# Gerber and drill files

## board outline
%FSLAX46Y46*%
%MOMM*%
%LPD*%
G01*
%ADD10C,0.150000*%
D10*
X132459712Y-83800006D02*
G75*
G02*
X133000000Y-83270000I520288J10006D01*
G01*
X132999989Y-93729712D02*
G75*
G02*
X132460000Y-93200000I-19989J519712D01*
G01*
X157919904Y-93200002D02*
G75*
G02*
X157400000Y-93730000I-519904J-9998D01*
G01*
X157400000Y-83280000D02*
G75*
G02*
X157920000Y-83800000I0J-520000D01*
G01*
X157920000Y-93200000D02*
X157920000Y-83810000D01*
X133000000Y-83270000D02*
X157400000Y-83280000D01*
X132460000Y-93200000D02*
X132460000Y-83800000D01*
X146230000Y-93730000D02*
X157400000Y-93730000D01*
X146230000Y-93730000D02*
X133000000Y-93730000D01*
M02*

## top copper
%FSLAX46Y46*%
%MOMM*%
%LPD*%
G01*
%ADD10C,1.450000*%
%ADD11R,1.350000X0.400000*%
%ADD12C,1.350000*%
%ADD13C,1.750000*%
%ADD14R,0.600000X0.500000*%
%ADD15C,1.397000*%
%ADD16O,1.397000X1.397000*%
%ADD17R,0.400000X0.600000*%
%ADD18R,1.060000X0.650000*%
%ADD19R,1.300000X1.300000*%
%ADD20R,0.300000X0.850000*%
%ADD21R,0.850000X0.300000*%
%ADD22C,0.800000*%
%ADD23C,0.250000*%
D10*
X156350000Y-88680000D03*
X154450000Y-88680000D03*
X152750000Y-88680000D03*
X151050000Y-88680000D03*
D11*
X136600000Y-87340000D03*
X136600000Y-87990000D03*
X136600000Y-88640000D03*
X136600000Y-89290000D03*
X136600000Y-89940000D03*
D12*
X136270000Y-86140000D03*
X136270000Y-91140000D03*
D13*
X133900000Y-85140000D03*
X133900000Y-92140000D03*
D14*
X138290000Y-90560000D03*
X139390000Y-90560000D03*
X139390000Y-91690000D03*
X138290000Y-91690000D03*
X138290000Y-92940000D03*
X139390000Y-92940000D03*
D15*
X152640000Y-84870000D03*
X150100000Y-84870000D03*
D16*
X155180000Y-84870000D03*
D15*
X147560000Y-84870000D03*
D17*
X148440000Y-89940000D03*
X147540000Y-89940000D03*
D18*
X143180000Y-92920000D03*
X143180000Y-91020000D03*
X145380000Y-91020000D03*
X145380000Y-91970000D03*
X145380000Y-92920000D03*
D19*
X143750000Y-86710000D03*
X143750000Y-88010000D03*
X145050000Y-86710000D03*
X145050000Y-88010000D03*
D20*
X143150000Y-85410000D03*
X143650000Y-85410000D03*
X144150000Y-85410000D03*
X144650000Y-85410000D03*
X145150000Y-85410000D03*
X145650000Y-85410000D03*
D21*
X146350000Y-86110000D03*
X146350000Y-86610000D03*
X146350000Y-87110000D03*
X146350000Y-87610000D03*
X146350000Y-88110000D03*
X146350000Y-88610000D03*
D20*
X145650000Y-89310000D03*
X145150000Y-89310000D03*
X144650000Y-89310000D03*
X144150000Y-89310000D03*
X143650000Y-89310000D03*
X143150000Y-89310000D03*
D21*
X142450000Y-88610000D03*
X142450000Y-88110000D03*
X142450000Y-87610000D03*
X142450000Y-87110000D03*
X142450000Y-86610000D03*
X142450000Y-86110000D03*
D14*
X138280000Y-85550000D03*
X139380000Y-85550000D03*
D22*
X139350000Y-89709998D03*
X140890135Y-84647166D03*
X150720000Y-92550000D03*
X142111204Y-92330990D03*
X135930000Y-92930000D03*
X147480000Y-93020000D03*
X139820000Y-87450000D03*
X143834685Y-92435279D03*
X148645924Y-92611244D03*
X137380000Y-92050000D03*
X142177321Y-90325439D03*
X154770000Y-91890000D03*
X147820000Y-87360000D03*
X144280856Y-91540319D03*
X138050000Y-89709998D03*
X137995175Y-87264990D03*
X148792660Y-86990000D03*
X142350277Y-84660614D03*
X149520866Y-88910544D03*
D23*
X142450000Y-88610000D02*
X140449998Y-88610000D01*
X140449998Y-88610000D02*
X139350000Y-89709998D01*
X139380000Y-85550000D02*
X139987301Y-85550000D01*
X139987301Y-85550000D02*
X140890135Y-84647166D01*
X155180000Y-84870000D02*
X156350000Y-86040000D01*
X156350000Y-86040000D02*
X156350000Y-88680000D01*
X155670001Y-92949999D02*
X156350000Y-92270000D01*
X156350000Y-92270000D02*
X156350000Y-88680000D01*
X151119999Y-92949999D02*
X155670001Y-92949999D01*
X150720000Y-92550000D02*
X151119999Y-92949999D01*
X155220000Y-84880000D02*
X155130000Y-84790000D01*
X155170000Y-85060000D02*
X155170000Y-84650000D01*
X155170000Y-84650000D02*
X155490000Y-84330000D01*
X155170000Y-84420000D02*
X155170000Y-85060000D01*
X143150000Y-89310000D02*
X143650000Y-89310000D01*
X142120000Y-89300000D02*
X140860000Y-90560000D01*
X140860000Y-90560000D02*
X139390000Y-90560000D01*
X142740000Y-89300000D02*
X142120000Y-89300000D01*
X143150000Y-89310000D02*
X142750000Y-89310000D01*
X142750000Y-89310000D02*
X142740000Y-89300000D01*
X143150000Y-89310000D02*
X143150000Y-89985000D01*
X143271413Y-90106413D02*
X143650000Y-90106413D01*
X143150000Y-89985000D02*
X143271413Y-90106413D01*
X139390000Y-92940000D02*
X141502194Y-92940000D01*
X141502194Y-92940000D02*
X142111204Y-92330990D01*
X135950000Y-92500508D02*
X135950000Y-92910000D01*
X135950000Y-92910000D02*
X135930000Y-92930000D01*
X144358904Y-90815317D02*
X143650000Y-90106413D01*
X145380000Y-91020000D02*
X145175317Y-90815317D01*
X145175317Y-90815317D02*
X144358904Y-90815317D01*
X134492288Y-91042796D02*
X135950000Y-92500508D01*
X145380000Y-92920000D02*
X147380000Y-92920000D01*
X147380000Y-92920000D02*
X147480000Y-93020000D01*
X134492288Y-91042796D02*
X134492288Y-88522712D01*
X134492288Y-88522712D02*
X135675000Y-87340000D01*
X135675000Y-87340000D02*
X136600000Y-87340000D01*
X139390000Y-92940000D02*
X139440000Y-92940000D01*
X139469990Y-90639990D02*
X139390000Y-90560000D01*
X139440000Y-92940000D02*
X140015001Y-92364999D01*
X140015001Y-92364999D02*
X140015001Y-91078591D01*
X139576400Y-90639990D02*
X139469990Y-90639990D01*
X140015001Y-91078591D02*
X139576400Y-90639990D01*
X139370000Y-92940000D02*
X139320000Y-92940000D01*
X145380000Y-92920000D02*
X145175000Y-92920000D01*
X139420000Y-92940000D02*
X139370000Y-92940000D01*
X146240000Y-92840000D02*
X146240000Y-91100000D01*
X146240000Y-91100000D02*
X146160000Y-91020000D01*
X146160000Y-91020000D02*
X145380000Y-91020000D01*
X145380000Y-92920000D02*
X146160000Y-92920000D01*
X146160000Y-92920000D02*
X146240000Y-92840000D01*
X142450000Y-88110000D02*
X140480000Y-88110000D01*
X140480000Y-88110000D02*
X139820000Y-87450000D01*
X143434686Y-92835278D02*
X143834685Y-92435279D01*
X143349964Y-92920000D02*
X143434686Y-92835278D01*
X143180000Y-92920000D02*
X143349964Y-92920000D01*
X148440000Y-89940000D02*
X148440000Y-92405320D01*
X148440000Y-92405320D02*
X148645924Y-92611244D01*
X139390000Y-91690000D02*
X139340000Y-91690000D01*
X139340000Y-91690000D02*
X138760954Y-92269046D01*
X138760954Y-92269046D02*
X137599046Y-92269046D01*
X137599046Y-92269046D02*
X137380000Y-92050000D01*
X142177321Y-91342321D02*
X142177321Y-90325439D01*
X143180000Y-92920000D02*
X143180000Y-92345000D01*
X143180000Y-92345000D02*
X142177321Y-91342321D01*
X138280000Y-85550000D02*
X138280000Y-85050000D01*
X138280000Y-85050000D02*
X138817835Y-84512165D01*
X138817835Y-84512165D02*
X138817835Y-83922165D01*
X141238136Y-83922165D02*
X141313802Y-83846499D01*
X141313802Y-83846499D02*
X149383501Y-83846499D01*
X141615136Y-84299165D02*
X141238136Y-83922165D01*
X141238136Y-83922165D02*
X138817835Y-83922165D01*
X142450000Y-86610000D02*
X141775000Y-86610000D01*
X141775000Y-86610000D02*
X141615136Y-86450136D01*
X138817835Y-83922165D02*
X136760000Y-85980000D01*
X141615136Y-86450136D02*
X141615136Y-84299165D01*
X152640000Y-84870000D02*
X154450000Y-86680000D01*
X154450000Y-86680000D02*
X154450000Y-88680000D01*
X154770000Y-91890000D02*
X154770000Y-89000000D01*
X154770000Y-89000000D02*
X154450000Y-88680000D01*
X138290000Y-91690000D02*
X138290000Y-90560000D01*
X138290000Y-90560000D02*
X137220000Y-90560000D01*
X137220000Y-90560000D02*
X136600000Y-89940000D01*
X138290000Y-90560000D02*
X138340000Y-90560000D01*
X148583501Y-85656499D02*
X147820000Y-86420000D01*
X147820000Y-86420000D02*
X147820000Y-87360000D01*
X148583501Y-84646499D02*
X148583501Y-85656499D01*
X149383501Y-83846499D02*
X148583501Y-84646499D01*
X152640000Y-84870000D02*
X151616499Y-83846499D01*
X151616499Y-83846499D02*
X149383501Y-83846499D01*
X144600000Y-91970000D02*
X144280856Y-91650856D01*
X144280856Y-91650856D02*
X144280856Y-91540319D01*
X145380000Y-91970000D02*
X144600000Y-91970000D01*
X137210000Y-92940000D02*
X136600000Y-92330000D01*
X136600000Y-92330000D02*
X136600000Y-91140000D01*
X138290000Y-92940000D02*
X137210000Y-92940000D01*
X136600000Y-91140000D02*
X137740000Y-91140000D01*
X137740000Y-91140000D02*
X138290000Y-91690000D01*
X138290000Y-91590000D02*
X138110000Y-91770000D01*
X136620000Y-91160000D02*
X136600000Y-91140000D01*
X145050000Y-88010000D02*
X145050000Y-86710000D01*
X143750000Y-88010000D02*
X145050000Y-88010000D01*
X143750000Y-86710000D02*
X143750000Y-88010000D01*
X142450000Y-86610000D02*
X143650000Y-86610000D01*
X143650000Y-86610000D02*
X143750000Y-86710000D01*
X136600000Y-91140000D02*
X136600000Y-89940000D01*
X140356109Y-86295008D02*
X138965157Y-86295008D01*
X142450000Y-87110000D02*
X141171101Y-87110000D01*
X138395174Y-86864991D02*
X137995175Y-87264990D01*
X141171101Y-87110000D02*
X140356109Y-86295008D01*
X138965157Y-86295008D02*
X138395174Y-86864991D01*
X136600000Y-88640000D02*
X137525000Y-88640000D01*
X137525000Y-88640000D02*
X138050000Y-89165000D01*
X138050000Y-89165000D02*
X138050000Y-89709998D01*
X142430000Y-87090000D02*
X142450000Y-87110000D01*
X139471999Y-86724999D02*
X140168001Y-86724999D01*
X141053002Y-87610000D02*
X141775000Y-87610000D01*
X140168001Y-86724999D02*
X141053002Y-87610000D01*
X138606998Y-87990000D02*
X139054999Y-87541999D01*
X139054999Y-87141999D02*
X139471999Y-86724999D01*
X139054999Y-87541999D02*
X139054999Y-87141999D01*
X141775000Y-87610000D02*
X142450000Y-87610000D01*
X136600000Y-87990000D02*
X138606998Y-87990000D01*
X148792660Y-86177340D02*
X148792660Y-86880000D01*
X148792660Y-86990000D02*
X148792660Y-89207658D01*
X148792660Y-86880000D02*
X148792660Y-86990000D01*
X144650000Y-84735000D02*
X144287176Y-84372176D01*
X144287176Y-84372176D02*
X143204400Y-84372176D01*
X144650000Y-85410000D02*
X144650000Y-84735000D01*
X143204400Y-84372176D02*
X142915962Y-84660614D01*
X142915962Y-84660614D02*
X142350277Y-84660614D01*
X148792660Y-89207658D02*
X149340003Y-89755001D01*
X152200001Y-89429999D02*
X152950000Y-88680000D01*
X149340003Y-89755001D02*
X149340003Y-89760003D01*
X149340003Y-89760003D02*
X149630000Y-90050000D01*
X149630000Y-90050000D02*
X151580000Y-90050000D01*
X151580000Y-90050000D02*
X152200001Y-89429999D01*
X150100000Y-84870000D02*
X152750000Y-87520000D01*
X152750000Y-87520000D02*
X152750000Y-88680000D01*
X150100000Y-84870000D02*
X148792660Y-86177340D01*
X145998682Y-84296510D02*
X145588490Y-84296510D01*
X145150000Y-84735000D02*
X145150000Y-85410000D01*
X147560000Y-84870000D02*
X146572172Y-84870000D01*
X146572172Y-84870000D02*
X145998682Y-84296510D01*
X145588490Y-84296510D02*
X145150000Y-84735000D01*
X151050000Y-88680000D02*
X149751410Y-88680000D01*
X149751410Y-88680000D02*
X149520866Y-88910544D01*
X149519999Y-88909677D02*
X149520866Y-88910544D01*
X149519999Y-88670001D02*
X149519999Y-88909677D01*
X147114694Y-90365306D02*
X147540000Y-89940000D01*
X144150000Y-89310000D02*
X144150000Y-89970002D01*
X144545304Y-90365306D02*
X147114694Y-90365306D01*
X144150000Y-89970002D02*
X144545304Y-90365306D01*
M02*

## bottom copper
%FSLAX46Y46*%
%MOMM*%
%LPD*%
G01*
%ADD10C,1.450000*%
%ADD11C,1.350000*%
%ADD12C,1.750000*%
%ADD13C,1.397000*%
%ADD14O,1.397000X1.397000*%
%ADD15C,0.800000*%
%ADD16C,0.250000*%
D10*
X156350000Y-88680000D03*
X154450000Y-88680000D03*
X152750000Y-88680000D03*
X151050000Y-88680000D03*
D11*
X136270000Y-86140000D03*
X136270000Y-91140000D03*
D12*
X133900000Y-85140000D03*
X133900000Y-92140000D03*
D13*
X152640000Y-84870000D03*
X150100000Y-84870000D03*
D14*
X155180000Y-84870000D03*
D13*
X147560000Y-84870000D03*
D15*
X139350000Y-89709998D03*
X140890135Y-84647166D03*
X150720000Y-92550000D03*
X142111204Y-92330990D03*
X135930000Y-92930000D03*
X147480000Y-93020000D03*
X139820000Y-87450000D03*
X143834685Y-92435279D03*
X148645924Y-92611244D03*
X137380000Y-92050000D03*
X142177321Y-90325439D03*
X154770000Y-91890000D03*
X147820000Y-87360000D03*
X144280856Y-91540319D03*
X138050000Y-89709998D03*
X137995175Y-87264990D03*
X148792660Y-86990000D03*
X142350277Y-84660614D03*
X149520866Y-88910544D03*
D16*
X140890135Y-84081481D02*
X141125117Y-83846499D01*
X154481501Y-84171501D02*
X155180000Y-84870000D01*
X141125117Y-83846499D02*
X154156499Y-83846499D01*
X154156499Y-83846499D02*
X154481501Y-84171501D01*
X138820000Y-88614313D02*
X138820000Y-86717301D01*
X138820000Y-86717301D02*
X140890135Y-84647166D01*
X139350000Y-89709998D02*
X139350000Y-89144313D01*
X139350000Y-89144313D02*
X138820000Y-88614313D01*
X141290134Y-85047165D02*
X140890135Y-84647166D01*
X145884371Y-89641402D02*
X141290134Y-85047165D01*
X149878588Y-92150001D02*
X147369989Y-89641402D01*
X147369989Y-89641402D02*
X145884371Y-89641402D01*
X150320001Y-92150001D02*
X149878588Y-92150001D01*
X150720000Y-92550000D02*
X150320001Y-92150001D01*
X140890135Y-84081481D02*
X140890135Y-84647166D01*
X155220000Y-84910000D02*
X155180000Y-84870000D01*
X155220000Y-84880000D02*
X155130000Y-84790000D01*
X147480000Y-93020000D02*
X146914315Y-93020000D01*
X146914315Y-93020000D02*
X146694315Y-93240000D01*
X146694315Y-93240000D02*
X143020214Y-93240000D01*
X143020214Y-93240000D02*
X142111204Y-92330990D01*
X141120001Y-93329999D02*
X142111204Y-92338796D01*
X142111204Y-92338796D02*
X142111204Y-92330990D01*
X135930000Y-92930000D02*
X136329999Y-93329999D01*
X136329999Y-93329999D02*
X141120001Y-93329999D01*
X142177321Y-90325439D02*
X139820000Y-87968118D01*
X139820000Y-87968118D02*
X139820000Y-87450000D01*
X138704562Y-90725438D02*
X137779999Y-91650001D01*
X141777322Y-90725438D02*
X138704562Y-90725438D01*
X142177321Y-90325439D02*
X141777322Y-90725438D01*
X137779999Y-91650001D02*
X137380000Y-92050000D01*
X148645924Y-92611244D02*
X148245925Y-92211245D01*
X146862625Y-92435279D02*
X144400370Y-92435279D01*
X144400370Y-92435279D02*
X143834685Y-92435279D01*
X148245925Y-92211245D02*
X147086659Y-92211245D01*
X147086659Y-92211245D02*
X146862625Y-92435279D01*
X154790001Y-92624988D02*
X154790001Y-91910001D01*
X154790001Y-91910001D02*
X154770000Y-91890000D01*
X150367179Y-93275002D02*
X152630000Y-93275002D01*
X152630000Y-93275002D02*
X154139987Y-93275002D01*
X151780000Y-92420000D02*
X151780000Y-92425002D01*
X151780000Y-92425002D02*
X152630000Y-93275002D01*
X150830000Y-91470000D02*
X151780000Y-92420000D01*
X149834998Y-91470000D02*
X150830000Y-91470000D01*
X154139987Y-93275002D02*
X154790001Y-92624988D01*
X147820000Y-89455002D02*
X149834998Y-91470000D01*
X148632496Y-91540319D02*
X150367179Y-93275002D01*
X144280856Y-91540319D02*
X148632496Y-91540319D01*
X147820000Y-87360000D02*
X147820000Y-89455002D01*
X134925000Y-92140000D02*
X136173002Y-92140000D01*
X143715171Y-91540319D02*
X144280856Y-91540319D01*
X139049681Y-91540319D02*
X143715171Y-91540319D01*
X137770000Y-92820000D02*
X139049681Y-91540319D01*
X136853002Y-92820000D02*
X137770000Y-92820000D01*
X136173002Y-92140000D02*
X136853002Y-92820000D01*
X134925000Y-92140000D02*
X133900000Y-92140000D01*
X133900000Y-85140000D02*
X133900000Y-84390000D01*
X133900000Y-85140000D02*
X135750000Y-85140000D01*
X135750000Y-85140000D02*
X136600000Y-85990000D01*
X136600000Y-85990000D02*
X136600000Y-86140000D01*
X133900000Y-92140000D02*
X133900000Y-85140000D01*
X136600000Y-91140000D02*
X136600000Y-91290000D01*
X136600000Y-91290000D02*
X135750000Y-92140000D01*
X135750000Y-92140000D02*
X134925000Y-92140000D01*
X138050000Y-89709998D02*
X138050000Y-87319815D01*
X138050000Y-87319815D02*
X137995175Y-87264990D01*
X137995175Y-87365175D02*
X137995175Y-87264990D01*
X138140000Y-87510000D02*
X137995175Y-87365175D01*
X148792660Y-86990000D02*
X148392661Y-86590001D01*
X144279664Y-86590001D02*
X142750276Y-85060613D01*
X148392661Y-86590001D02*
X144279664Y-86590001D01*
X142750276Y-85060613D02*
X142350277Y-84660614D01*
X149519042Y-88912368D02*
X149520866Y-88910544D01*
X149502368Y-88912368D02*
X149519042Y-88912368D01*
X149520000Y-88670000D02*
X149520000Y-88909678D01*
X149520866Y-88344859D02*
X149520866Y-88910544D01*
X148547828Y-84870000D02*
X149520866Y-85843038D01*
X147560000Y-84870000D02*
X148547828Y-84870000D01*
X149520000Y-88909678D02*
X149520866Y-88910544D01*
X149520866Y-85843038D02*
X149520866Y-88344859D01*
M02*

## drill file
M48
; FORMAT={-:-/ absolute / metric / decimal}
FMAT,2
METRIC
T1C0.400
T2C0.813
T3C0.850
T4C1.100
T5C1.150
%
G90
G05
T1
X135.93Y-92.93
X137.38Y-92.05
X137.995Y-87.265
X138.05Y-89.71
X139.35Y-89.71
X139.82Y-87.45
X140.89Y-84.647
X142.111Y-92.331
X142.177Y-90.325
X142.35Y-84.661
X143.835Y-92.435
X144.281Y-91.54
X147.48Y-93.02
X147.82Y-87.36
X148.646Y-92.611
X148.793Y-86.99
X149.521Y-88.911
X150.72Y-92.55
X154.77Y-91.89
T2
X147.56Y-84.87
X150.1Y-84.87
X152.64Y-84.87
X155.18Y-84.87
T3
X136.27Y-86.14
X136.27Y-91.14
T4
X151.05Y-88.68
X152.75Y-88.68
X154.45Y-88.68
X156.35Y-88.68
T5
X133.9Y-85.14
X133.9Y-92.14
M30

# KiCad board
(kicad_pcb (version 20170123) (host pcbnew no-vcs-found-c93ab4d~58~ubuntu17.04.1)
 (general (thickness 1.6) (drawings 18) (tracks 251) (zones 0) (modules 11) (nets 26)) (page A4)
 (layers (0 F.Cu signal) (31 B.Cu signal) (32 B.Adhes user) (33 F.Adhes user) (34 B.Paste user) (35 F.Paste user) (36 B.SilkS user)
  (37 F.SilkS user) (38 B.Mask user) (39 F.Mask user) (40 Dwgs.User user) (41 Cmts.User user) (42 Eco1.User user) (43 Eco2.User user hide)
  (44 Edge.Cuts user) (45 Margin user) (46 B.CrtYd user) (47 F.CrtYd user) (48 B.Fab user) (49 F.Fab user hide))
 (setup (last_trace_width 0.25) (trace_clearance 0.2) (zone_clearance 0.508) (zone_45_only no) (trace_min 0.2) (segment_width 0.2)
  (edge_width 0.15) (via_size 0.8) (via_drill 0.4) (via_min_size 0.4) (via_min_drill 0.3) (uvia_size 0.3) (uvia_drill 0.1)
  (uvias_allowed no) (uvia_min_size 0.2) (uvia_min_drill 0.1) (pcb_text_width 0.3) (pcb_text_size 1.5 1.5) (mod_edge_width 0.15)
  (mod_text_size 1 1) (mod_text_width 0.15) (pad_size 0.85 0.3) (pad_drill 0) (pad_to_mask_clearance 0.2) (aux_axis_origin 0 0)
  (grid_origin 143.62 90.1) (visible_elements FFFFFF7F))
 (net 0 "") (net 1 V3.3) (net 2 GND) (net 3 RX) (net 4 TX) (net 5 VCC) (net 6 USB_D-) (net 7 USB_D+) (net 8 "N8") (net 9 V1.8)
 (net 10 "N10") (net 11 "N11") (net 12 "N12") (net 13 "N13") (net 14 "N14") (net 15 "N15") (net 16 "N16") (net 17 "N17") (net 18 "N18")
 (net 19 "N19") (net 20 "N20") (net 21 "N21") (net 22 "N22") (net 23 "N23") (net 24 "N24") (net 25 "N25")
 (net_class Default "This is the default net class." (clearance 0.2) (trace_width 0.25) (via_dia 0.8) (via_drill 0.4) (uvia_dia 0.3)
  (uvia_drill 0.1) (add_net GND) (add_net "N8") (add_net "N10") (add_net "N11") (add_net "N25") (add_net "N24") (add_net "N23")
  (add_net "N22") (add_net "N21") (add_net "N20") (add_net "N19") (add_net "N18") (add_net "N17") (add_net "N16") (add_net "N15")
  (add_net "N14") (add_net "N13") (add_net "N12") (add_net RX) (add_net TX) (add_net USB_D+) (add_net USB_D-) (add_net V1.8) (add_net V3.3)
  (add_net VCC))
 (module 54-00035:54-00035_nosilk (layer F.Cu) (at 149.1 88.68)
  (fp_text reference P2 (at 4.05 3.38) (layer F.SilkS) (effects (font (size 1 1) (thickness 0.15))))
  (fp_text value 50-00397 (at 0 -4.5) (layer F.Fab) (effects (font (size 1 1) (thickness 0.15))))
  (pad 4 thru_hole circle (at 7.25 0) (size 1.45 1.45) (drill 1.1) (layers *.Cu *.Mask) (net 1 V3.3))
  (pad 3 thru_hole circle (at 5.35 0) (size 1.45 1.45) (drill 1.1) (layers *.Cu *.Mask) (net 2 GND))
  (pad 2 thru_hole circle (at 3.65 0) (size 1.45 1.45) (drill 1.1) (layers *.Cu *.Mask) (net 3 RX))
  (pad 1 thru_hole circle (at 1.95 0) (size 1.45 1.45) (drill 1.1) (layers *.Cu *.Mask) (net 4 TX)))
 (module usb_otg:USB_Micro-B (layer F.Cu) (at 135.25 88.64 270)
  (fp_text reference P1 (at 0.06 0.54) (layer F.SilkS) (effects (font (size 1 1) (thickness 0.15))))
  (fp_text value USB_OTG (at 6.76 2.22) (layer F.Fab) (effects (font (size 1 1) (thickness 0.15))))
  (pad 1 smd rect (at -1.3 -1.35) (size 1.35 0.4) (layers F.Cu F.Paste F.Mask) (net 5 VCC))
  (pad 2 smd rect (at -0.65 -1.35) (size 1.35 0.4) (layers F.Cu F.Paste F.Mask) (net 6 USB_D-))
  (pad 3 smd rect (at 0 -1.35) (size 1.35 0.4) (layers F.Cu F.Paste F.Mask) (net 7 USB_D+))
  (pad 4 smd rect (at 0.65 -1.35) (size 1.35 0.4) (layers F.Cu F.Paste F.Mask) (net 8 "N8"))
  (pad 5 smd rect (at 1.3 -1.35) (size 1.35 0.4) (layers F.Cu F.Paste F.Mask) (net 2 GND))
  (pad 6 thru_hole circle (at -2.5 -1.02) (size 1.35 1.35) (drill 0.85) (layers *.Cu *.Mask) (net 2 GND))
  (pad 6 thru_hole circle (at 2.5 -1.02) (size 1.35 1.35) (drill 0.85) (layers *.Cu *.Mask) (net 2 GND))
  (pad 6 thru_hole circle (at -3.5 1.35) (size 1.75 1.75) (drill 1.15) (layers *.Cu *.Mask) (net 2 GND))
  (pad 6 thru_hole circle (at 3.5 1.35) (size 1.75 1.75) (drill 1.15) (layers *.Cu *.Mask) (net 2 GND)))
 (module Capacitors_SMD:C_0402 (layer F.Cu) (at 138.84 90.56)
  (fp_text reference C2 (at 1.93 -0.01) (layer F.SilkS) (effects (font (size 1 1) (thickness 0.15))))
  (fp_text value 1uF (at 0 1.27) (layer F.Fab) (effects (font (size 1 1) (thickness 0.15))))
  (pad 1 smd rect (at -0.55 0) (size 0.6 0.5) (layers F.Cu F.Paste F.Mask) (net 2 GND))
  (pad 2 smd rect (at 0.55 0) (size 0.6 0.5) (layers F.Cu F.Paste F.Mask) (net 5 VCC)))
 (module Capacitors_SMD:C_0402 (layer F.Cu) (at 138.84 91.69 180)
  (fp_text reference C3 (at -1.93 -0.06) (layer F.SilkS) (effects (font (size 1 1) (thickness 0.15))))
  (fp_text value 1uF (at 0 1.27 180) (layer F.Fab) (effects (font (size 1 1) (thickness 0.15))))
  (pad 1 smd rect (at -0.55 0 180) (size 0.6 0.5) (layers F.Cu F.Paste F.Mask) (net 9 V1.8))
  (pad 2 smd rect (at 0.55 0 180) (size 0.6 0.5) (layers F.Cu F.Paste F.Mask) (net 2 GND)))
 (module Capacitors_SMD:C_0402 (layer F.Cu) (at 138.84 92.94 180)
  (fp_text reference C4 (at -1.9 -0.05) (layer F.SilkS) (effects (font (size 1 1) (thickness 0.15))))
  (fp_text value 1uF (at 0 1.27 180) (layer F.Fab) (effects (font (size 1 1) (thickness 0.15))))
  (pad 2 smd rect (at 0.55 0 180) (size 0.6 0.5) (layers F.Cu F.Paste F.Mask) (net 2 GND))
  (pad 1 smd rect (at -0.55 0 180) (size 0.6 0.5) (layers F.Cu F.Paste F.Mask) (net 5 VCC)))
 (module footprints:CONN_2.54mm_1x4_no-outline (layer F.Cu) (at 151.37 84.87)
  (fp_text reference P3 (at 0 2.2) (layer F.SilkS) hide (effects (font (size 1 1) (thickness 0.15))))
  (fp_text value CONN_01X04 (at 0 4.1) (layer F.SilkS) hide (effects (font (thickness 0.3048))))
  (pad 2 thru_hole circle (at 1.27 0) (size 1.397 1.397) (drill 0.8128) (layers *.Cu *.Mask F.SilkS) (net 2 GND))
  (pad 3 thru_hole circle (at -1.27 0) (size 1.397 1.397) (drill 0.8128) (layers *.Cu *.Mask F.SilkS) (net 3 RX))
  (pad 1 thru_hole oval (at 3.81 0) (size 1.397 1.397) (drill 0.8128) (layers *.Cu *.Mask F.SilkS) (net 1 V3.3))
  (pad 4 thru_hole circle (at -3.81 0) (size 1.397 1.397) (drill 0.8128) (layers *.Cu *.Mask F.SilkS) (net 4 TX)))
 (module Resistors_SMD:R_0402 (layer F.Cu) (at 147.99 89.94)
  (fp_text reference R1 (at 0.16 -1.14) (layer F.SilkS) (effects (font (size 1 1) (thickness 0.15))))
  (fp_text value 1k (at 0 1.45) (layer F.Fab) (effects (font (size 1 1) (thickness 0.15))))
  (pad 2 smd rect (at 0.45 0) (size 0.4 0.6) (layers F.Cu F.Paste F.Mask) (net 9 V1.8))
  (pad 1 smd rect (at -0.45 0) (size 0.4 0.6) (layers F.Cu F.Paste F.Mask) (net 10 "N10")))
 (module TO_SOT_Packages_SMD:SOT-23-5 (layer F.Cu) (at 144.28 91.97 180)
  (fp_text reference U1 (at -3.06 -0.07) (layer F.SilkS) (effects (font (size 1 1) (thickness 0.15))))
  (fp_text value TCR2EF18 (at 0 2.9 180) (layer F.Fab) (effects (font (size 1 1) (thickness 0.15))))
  (pad 5 smd rect (at 1.1 -0.95 180) (size 1.06 0.65) (layers F.Cu F.Paste F.Mask) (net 9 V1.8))
  (pad 4 smd rect (at 1.1 0.95 180) (size 1.06 0.65) (layers F.Cu F.Paste F.Mask) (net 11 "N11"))
  (pad 3 smd rect (at -1.1 0.95 180) (size 1.06 0.65) (layers F.Cu F.Paste F.Mask) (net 5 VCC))
  (pad 2 smd rect (at -1.1 0 180) (size 1.06 0.65) (layers F.Cu F.Paste F.Mask) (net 2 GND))
  (pad 1 smd rect (at -1.1 -0.95 180) (size 1.06 0.65) (layers F.Cu F.Paste F.Mask) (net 5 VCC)))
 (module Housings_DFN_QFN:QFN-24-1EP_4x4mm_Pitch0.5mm (layer F.Cu) (at 144.4 87.36)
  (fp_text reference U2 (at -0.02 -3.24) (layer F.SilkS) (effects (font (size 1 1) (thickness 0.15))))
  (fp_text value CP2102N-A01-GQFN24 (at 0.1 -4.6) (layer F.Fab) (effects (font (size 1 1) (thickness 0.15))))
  (pad 25 smd rect (at -0.65 -0.65) (size 1.3 1.3) (layers F.Cu F.Paste F.Mask) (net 2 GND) (solder_paste_margin_ratio -0.2))
  (pad 25 smd rect (at -0.65 0.65) (size 1.3 1.3) (layers F.Cu F.Paste F.Mask) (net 2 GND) (solder_paste_margin_ratio -0.2))
  (pad 25 smd rect (at 0.65 -0.65) (size 1.3 1.3) (layers F.Cu F.Paste F.Mask) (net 2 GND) (solder_paste_margin_ratio -0.2))
  (pad 25 smd rect (at 0.65 0.65) (size 1.3 1.3) (layers F.Cu F.Paste F.Mask) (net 2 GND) (solder_paste_margin_ratio -0.2))
  (pad 24 smd rect (at -1.25 -1.95 90) (size 0.85 0.3) (layers F.Cu F.Paste F.Mask) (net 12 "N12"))
  (pad 23 smd rect (at -0.75 -1.95 90) (size 0.85 0.3) (layers F.Cu F.Paste F.Mask) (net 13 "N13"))
  (pad 22 smd rect (at -0.25 -1.95 90) (size 0.85 0.3) (layers F.Cu F.Paste F.Mask) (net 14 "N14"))
  (pad 21 smd rect (at 0.25 -1.95 90) (size 0.85 0.3) (layers F.Cu F.Paste F.Mask) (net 3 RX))
  (pad 20 smd rect (at 0.75 -1.95 90) (size 0.85 0.3) (layers F.Cu F.Paste F.Mask) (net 4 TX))
  (pad 19 smd rect (at 1.25 -1.95 90) (size 0.85 0.3) (layers F.Cu F.Paste F.Mask) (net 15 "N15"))
  (pad 18 smd rect (at 1.95 -1.25) (size 0.85 0.3) (layers F.Cu F.Paste F.Mask) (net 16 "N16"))
  (pad 17 smd rect (at 1.95 -0.75) (size 0.85 0.3) (layers F.Cu F.Paste F.Mask) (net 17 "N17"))
  (pad 16 smd rect (at 1.95 -0.25) (size 0.85 0.3) (layers F.Cu F.Paste F.Mask) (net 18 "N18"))
  (pad 15 smd rect (at 1.95 0.25) (size 0.85 0.3) (layers F.Cu F.Paste F.Mask) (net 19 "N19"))
  (pad 14 smd rect (at 1.95 0.75) (size 0.85 0.3) (layers F.Cu F.Paste F.Mask) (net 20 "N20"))
  (pad 13 smd rect (at 1.95 1.25) (size 0.85 0.3) (layers F.Cu F.Paste F.Mask) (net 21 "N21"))
  (pad 12 smd rect (at 1.25 1.95 90) (size 0.85 0.3) (layers F.Cu F.Paste F.Mask) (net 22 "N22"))
  (pad 11 smd rect (at 0.75 1.95 90) (size 0.85 0.3) (layers F.Cu F.Paste F.Mask) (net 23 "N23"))
  (pad 10 smd rect (at 0.25 1.95 90) (size 0.85 0.3) (layers F.Cu F.Paste F.Mask) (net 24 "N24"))
  (pad 9 smd rect (at -0.25 1.95 90) (size 0.85 0.3) (layers F.Cu F.Paste F.Mask) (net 10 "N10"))
  (pad 8 smd rect (at -0.75 1.95 90) (size 0.85 0.3) (layers F.Cu F.Paste F.Mask) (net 5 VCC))
  (pad 7 smd rect (at -1.25 1.95 90) (size 0.85 0.3) (layers F.Cu F.Paste F.Mask) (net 5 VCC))
  (pad 6 smd rect (at -1.95 1.25) (size 0.85 0.3) (layers F.Cu F.Paste F.Mask) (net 1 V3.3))
  (pad 5 smd rect (at -1.95 0.75) (size 0.85 0.3) (layers F.Cu F.Paste F.Mask) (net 9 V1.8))
  (pad 4 smd rect (at -1.95 0.25) (size 0.85 0.3) (layers F.Cu F.Paste F.Mask) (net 6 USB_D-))
  (pad 3 smd rect (at -1.95 -0.25) (size 0.85 0.3) (layers F.Cu F.Paste F.Mask) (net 7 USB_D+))
  (pad 2 smd rect (at -1.95 -0.75) (size 0.85 0.3) (layers F.Cu F.Paste F.Mask) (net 2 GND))
  (pad 1 smd rect (at -1.95 -1.25) (size 0.85 0.3) (layers F.Cu F.Paste F.Mask) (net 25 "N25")))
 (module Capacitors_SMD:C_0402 (layer F.Cu) (at 138.83 85.55 180)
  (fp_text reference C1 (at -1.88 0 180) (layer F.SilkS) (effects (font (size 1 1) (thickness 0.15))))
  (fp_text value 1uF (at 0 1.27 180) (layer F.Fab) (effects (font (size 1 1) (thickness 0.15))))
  (pad 2 smd rect (at 0.55 0 180) (size 0.6 0.5) (layers F.Cu F.Paste F.Mask) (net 2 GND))
  (pad 1 smd rect (at -0.55 0 180) (size 0.6 0.5) (layers F.Cu F.Paste F.Mask) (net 1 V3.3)))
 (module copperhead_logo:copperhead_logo (layer B.Cu) (at 141.43 88.4)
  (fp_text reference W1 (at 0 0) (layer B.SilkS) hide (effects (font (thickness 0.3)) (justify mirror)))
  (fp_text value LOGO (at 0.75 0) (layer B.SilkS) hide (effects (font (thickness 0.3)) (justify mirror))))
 (gr_arc (start 132.98 83.79) (end 133 83.27) (angle -93.30435508) (layer Edge.Cuts) (width 0.15))
 (gr_arc (start 132.98 93.21) (end 132.46 93.2) (angle -93.30431274) (layer Edge.Cuts) (width 0.15))
 (gr_arc (start 157.4 93.21) (end 157.4 93.73) (angle -91.10169129) (layer Edge.Cuts) (width 0.15))
 (gr_arc (start 157.4 83.8) (end 157.92 83.8) (angle -90) (layer Edge.Cuts) (width 0.15))
 (gr_line (start 157.92 93.2) (end 157.92 83.81) (layer Edge.Cuts) (width 0.15))
 (gr_line (start 133 83.27) (end 157.4 83.28) (layer Edge.Cuts) (width 0.15))
 (gr_line (start 132.46 93.2) (end 132.46 83.8) (layer Edge.Cuts) (width 0.15))
 (gr_line (start 146.23 93.73) (end 157.4 93.73) (layer Edge.Cuts) (width 0.15))
 (gr_line (start 146.23 93.73) (end 133 93.73) (layer Edge.Cuts) (width 0.15))
 (segment (start 140.890135 84.081481) (end 141.125117 83.846499) (width 0.25) (layer B.Cu) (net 1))
 (segment (start 154.481501 84.171501) (end 155.18 84.87) (width 0.25) (layer B.Cu) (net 1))
 (segment (start 141.125117 83.846499) (end 154.156499 83.846499) (width 0.25) (layer B.Cu) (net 1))
 (segment (start 154.156499 83.846499) (end 154.481501 84.171501) (width 0.25) (layer B.Cu) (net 1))
 (segment (start 138.82 88.614313) (end 138.82 86.717301) (width 0.25) (layer B.Cu) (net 1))
 (segment (start 138.82 86.717301) (end 140.890135 84.647166) (width 0.25) (layer B.Cu) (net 1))
 (segment (start 139.35 89.709998) (end 139.35 89.144313) (width 0.25) (layer B.Cu) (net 1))
 (segment (start 139.35 89.144313) (end 138.82 88.614313) (width 0.25) (layer B.Cu) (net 1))
 (segment (start 142.45 88.61) (end 140.449998 88.61) (width 0.25) (layer F.Cu) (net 1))
 (via (at 139.35 89.709998) (size 0.8) (drill 0.4) (layers F.Cu B.Cu) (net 1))
 (segment (start 140.449998 88.61) (end 139.35 89.709998) (width 0.25) (layer F.Cu) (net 1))
 (segment (start 139.38 85.55) (end 139.987301 85.55) (width 0.25) (layer F.Cu) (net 1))
 (segment (start 139.987301 85.55) (end 140.890135 84.647166) (width 0.25) (layer F.Cu) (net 1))
 (segment (start 155.18 84.87) (end 156.35 86.04) (width 0.25) (layer F.Cu) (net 1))
 (segment (start 156.35 86.04) (end 156.35 88.68) (width 0.25) (layer F.Cu) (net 1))
 (segment (start 155.670001 92.949999) (end 156.35 92.27) (width 0.25) (layer F.Cu) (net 1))
 (segment (start 156.35 92.27) (end 156.35 88.68) (width 0.25) (layer F.Cu) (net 1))
 (segment (start 151.119999 92.949999) (end 155.670001 92.949999) (width 0.25) (layer F.Cu) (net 1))
 (segment (start 150.72 92.55) (end 151.119999 92.949999) (width 0.25) (layer F.Cu) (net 1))
 (segment (start 141.290134 85.047165) (end 140.890135 84.647166) (width 0.25) (layer B.Cu) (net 1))
 (segment (start 145.884371 89.641402) (end 141.290134 85.047165) (width 0.25) (layer B.Cu) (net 1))
 (segment (start 149.878588 92.150001) (end 147.369989 89.641402) (width 0.25) (layer B.Cu) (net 1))
 (segment (start 147.369989 89.641402) (end 145.884371 89.641402) (width 0.25) (layer B.Cu) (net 1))
 (segment (start 150.320001 92.150001) (end 149.878588 92.150001) (width 0.25) (layer B.Cu) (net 1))
 (segment (start 150.72 92.55) (end 150.320001 92.150001) (width 0.25) (layer B.Cu) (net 1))
 (via (at 140.890135 84.647166) (size 0.8) (drill 0.4) (layers F.Cu B.Cu) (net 1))
 (segment (start 140.890135 84.081481) (end 140.890135 84.647166) (width 0.25) (layer B.Cu) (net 1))
 (via (at 150.72 92.55) (size 0.8) (drill 0.4) (layers F.Cu B.Cu) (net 1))
 (segment (start 155.22 84.91) (end 155.18 84.87) (width 0.25) (layer B.Cu) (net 1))
 (segment (start 155.22 84.88) (end 155.13 84.79) (width 0.25) (layer B.Cu) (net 1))
 (segment (start 155.22 84.88) (end 155.13 84.79) (width 0.25) (layer F.Cu) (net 1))
 (segment (start 155.17 85.06) (end 155.17 84.65) (width 0.25) (layer F.Cu) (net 1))
 (segment (start 155.17 84.65) (end 155.49 84.33) (width 0.25) (layer F.Cu) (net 1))
 (segment (start 155.17 84.42) (end 155.17 85.06) (width 0.25) (layer F.Cu) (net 1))
 (segment (start 143.15 89.31) (end 143.65 89.31) (width 0.25) (layer F.Cu) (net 5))
 (segment (start 142.12 89.3) (end 140.86 90.56) (width 0.25) (layer F.Cu) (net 5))
 (segment (start 140.86 90.56) (end 139.39 90.56) (width 0.25) (layer F.Cu) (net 5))
 (segment (start 142.74 89.3) (end 142.12 89.3) (width 0.25) (layer F.Cu) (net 5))
 (segment (start 143.15 89.31) (end 142.75 89.31) (width 0.25) (layer F.Cu) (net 5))
 (segment (start 142.75 89.31) (end 142.74 89.3) (width 0.25) (layer F.Cu) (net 5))
 (segment (start 143.15 89.31) (end 143.15 89.985) (width 0.25) (layer F.Cu) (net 5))
 (segment (start 143.271413 90.106413) (end 143.65 90.106413) (width 0.25) (layer F.Cu) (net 5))
 (segment (start 143.15 89.985) (end 143.271413 90.106413) (width 0.25) (layer F.Cu) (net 5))
 (segment (start 139.39 92.94) (end 141.502194 92.94) (width 0.25) (layer F.Cu) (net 5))
 (segment (start 141.502194 92.94) (end 142.111204 92.33099) (width 0.25) (layer F.Cu) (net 5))
 (segment (start 147.48 93.02) (end 146.914315 93.02) (width 0.25) (layer B.Cu) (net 5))
 (segment (start 146.914315 93.02) (end 146.694315 93.24) (width 0.25) (layer B.Cu) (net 5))
 (segment (start 146.694315 93.24) (end 143.020214 93.24) (width 0.25) (layer B.Cu) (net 5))
 (segment (start 143.020214 93.24) (end 142.111204 92.33099) (width 0.25) (layer B.Cu) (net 5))
 (segment (start 141.120001 93.329999) (end 142.111204 92.338796) (width 0.25) (layer B.Cu) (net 5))
 (segment (start 142.111204 92.338796) (end 142.111204 92.33099) (width 0.25) (layer B.Cu) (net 5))
 (via (at 142.111204 92.33099) (size 0.8) (drill 0.4) (layers F.Cu B.Cu) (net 5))
 (segment (start 135.93 92.93) (end 136.329999 93.329999) (width 0.25) (layer B.Cu) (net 5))
 (segment (start 136.329999 93.329999) (end 141.120001 93.329999) (width 0.25) (layer B.Cu) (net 5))
 (segment (start 135.95 92.500508) (end 135.95 92.91) (width 0.25) (layer F.Cu) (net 5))
 (segment (start 135.95 92.91) (end 135.93 92.93) (width 0.25) (layer F.Cu) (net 5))
 (via (at 135.93 92.93) (size 0.8) (drill 0.4) (layers F.Cu B.Cu) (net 5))
 (segment (start 144.358904 90.815317) (end 143.65 90.106413) (width 0.25) (layer F.Cu) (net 5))
 (segment (start 145.38 91.02) (end 145.175317 90.815317) (width 0.25) (layer F.Cu) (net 5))
 (segment (start 145.175317 90.815317) (end 144.358904 90.815317) (width 0.25) (layer F.Cu) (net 5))
 (segment (start 134.492288 91.042796) (end 135.95 92.500508) (width 0.25) (layer F.Cu) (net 5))
 (segment (start 145.38 92.92) (end 147.38 92.92) (width 0.25) (layer F.Cu) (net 5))
 (via (at 147.48 93.02) (size 0.8) (drill 0.4) (layers F.Cu B.Cu) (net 5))
 (segment (start 147.38 92.92) (end 147.48 93.02) (width 0.25) (layer F.Cu) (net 5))
 (segment (start 134.492288 91.042796) (end 134.492288 88.522712) (width 0.25) (layer F.Cu) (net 5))
 (segment (start 134.492288 88.522712) (end 135.675 87.34) (width 0.25) (layer F.Cu) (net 5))
 (segment (start 135.675 87.34) (end 136.6 87.34) (width 0.25) (layer F.Cu) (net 5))
 (segment (start 139.39 92.94) (end 139.44 92.94) (width 0.25) (layer F.Cu) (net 5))
 (segment (start 139.46999 90.63999) (end 139.39 90.56) (width 0.25) (layer F.Cu) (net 5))
 (segment (start 139.44 92.94) (end 140.015001 92.364999) (width 0.25) (layer F.Cu) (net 5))
 (segment (start 140.015001 92.364999) (end 140.015001 91.078591) (width 0.25) (layer F.Cu) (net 5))
 (segment (start 139.5764 90.63999) (end 139.46999 90.63999) (width 0.25) (layer F.Cu) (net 5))
 (segment (start 140.015001 91.078591) (end 139.5764 90.63999) (width 0.25) (layer F.Cu) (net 5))
 (segment (start 139.37 92.94) (end 139.32 92.94) (width 0.25) (layer F.Cu) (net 5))
 (segment (start 145.38 92.92) (end 145.175 92.92) (width 0.25) (layer F.Cu) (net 5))
 (segment (start 139.42 92.94) (end 139.37 92.94) (width 0.25) (layer F.Cu) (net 5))
 (segment (start 146.24 92.84) (end 146.24 91.1) (width 0.25) (layer F.Cu) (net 5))
 (segment (start 146.24 91.1) (end 146.16 91.02) (width 0.25) (layer F.Cu) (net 5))
 (segment (start 146.16 91.02) (end 145.38 91.02) (width 0.25) (layer F.Cu) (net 5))
 (segment (start 145.38 92.92) (end 146.16 92.92) (width 0.25) (layer F.Cu) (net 5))
 (segment (start 146.16 92.92) (end 146.24 92.84) (width 0.25) (layer F.Cu) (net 5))
 (segment (start 142.177321 90.325439) (end 139.82 87.968118) (width 0.25) (layer B.Cu) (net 9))
 (segment (start 139.82 87.968118) (end 139.82 87.45) (width 0.25) (layer B.Cu) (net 9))
 (segment (start 142.45 88.11) (end 140.48 88.11) (width 0.25) (layer F.Cu) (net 9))
 (segment (start 140.48 88.11) (end 139.82 87.45) (width 0.25) (layer F.Cu) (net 9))
 (via (at 139.82 87.45) (size 0.8) (drill 0.4) (layers F.Cu B.Cu) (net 9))
 (segment (start 138.704562 90.725438) (end 137.779999 91.650001) (width 0.25) (layer B.Cu) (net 9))
 (segment (start 141.777322 90.725438) (end 138.704562 90.725438) (width 0.25) (layer B.Cu) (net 9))
 (segment (start 142.177321 90.325439) (end 141.777322 90.725438) (width 0.25) (layer B.Cu) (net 9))
 (segment (start 137.779999 91.650001) (end 137.38 92.05) (width 0.25) (layer B.Cu) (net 9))
 (via (at 143.834685 92.435279) (size 0.8) (drill 0.4) (layers F.Cu B.Cu) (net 9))
 (segment (start 148.645924 92.611244) (end 148.245925 92.211245) (width 0.25) (layer B.Cu) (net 9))
 (segment (start 143.434686 92.835278) (end 143.834685 92.435279) (width 0.25) (layer F.Cu) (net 9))
 (segment (start 143.349964 92.92) (end 143.434686 92.835278) (width 0.25) (layer F.Cu) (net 9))
 (segment (start 146.862625 92.435279) (end 144.40037 92.435279) (width 0.25) (layer B.Cu) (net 9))
 (segment (start 143.18 92.92) (end 143.349964 92.92) (width 0.25) (layer F.Cu) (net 9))
 (segment (start 144.40037 92.435279) (end 143.834685 92.435279) (width 0.25) (layer B.Cu) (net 9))
 (segment (start 148.245925 92.211245) (end 147.086659 92.211245) (width 0.25) (layer B.Cu) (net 9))
 (segment (start 147.086659 92.211245) (end 146.862625 92.435279) (width 0.25) (layer B.Cu) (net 9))
 (segment (start 148.44 89.94) (end 148.44 92.40532) (width 0.25) (layer F.Cu) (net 9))
 (via (at 148.645924 92.611244) (size 0.8) (drill 0.4) (layers F.Cu B.Cu) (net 9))
 (segment (start 148.44 92.40532) (end 148.645924 92.611244) (width 0.25) (layer F.Cu) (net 9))
 (segment (start 139.39 91.69) (end 139.34 91.69) (width 0.25) (layer F.Cu) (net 9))
 (segment (start 139.34 91.69) (end 138.760954 92.269046) (width 0.25) (layer F.Cu) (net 9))
 (segment (start 138.760954 92.269046) (end 137.599046 92.269046) (width 0.25) (layer F.Cu) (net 9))
 (segment (start 137.599046 92.269046) (end 137.38 92.05) (width 0.25) (layer F.Cu) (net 9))
 (via (at 137.38 92.05) (size 0.8) (drill 0.4) (layers F.Cu B.Cu) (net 9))
 (via (at 142.177321 90.325439) (size 0.8) (drill 0.4) (layers F.Cu B.Cu) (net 9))
 (segment (start 142.177321 91.342321) (end 142.177321 90.325439) (width 0.25) (layer F.Cu) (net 9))
 (segment (start 143.18 92.92) (end 143.18 92.345) (width 0.25) (layer F.Cu) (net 9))
 (segment (start 143.18 92.345) (end 142.177321 91.342321) (width 0.25) (layer F.Cu) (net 9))
 (segment (start 138.28 85.55) (end 138.28 85.05) (width 0.25) (layer F.Cu) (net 2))
 (segment (start 138.28 85.05) (end 138.817835 84.512165) (width 0.25) (layer F.Cu) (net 2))
 (segment (start 138.817835 84.512165) (end 138.817835 83.922165) (width 0.25) (layer F.Cu) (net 2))
 (segment (start 141.238136 83.922165) (end 141.313802 83.846499) (width 0.25) (layer F.Cu) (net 2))
 (segment (start 141.313802 83.846499) (end 149.383501 83.846499) (width 0.25) (layer F.Cu) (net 2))
 (segment (start 141.615136 84.299165) (end 141.238136 83.922165) (width 0.25) (layer F.Cu) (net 2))
 (segment (start 141.238136 83.922165) (end 138.817835 83.922165) (width 0.25) (layer F.Cu) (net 2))
 (segment (start 142.45 86.61) (end 141.775 86.61) (width 0.25) (layer F.Cu) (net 2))
 (segment (start 141.775 86.61) (end 141.615136 86.450136) (width 0.25) (layer F.Cu) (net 2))
 (segment (start 138.817835 83.922165) (end 136.76 85.98) (width 0.25) (layer F.Cu) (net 2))
 (segment (start 141.615136 86.450136) (end 141.615136 84.299165) (width 0.25) (layer F.Cu) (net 2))
 (segment (start 152.64 84.87) (end 154.45 86.68) (width 0.25) (layer F.Cu) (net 2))
 (segment (start 154.45 86.68) (end 154.45 88.68) (width 0.25) (layer F.Cu) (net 2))
 (segment (start 154.77 91.89) (end 154.77 89) (width 0.25) (layer F.Cu) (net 2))
 (segment (start 154.77 89) (end 154.45 88.68) (width 0.25) (layer F.Cu) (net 2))
 (segment (start 154.790001 92.624988) (end 154.790001 91.910001) (width 0.25) (layer B.Cu) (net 2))
 (segment (start 154.790001 91.910001) (end 154.77 91.89) (width 0.25) (layer B.Cu) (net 2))
 (via (at 154.77 91.89) (size 0.8) (drill 0.4) (layers F.Cu B.Cu) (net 2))
 (segment (start 138.29 91.69) (end 138.29 90.56) (width 0.25) (layer F.Cu) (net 2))
 (segment (start 138.29 90.56) (end 137.22 90.56) (width 0.25) (layer F.Cu) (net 2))
 (segment (start 137.22 90.56) (end 136.6 89.94) (width 0.25) (layer F.Cu) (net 2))
 (segment (start 138.29 90.56) (end 138.34 90.56) (width 0.25) (layer F.Cu) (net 2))
 (segment (start 150.367179 93.275002) (end 152.63 93.275002) (width 0.25) (layer B.Cu) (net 2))
 (segment (start 152.63 93.275002) (end 154.139987 93.275002) (width 0.25) (layer B.Cu) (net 2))
 (segment (start 151.78 92.42) (end 151.78 92.425002) (width 0.25) (layer B.Cu) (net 2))
 (segment (start 151.78 92.425002) (end 152.63 93.275002) (width 0.25) (layer B.Cu) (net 2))
 (segment (start 150.83 91.47) (end 151.78 92.42) (width 0.25) (layer B.Cu) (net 2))
 (segment (start 149.834998 91.47) (end 150.83 91.47) (width 0.25) (layer B.Cu) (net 2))
 (segment (start 154.139987 93.275002) (end 154.790001 92.624988) (width 0.25) (layer B.Cu) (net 2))
 (segment (start 147.82 89.455002) (end 149.834998 91.47) (width 0.25) (layer B.Cu) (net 2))
 (segment (start 148.632496 91.540319) (end 150.367179 93.275002) (width 0.25) (layer B.Cu) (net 2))
 (segment (start 144.280856 91.540319) (end 148.632496 91.540319) (width 0.25) (layer B.Cu) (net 2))
 (segment (start 147.82 87.36) (end 147.82 89.455002) (width 0.25) (layer B.Cu) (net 2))
 (segment (start 148.583501 85.656499) (end 147.82 86.42) (width 0.25) (layer F.Cu) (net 2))
 (segment (start 147.82 86.42) (end 147.82 87.36) (width 0.25) (layer F.Cu) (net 2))
 (via (at 147.82 87.36) (size 0.8) (drill 0.4) (layers F.Cu B.Cu) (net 2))
 (segment (start 148.583501 84.646499) (end 148.583501 85.656499) (width 0.25) (layer F.Cu) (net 2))
 (segment (start 149.383501 83.846499) (end 148.583501 84.646499) (width 0.25) (layer F.Cu) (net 2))
 (segment (start 152.64 84.87) (end 151.616499 83.846499) (width 0.25) (layer F.Cu) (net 2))
 (segment (start 151.616499 83.846499) (end 149.383501 83.846499) (width 0.25) (layer F.Cu) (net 2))
 (segment (start 144.6 91.97) (end 144.280856 91.650856) (width 0.25) (layer F.Cu) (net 2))
 (segment (start 144.280856 91.650856) (end 144.280856 91.540319) (width 0.25) (layer F.Cu) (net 2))
 (segment (start 145.38 91.97) (end 144.6 91.97) (width 0.25) (layer F.Cu) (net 2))
 (segment (start 134.925 92.14) (end 136.173002 92.14) (width 0.25) (layer B.Cu) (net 2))
 (segment (start 143.715171 91.540319) (end 144.280856 91.540319) (width 0.25) (layer B.Cu) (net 2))
 (segment (start 139.049681 91.540319) (end 143.715171 91.540319) (width 0.25) (layer B.Cu) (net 2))
 (segment (start 137.77 92.82) (end 139.049681 91.540319) (width 0.25) (layer B.Cu) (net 2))
 (segment (start 136.853002 92.82) (end 137.77 92.82) (width 0.25) (layer B.Cu) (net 2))
 (segment (start 136.173002 92.14) (end 136.853002 92.82) (width 0.25) (layer B.Cu) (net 2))
 (via (at 144.280856 91.540319) (size 0.8) (drill 0.4) (layers F.Cu B.Cu) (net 2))
 (segment (start 134.925 92.14) (end 133.9 92.14) (width 0.25) (layer B.Cu) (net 2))
 (segment (start 137.21 92.94) (end 136.6 92.33) (width 0.25) (layer F.Cu) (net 2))
 (segment (start 136.6 92.33) (end 136.6 91.14) (width 0.25) (layer F.Cu) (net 2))
 (segment (start 138.29 92.94) (end 137.21 92.94) (width 0.25) (layer F.Cu) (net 2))
 (segment (start 136.6 91.14) (end 137.74 91.14) (width 0.25) (layer F.Cu) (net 2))
 (segment (start 137.74 91.14) (end 138.29 91.69) (width 0.25) (layer F.Cu) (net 2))
 (segment (start 138.29 91.59) (end 138.11 91.77) (width 0.25) (layer F.Cu) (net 2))
 (segment (start 133.9 85.14) (end 133.9 84.39) (width 0.25) (layer B.Cu) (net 2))
 (segment (start 136.62 91.16) (end 136.6 91.14) (width 0.25) (layer F.Cu) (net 2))
 (segment (start 145.05 88.01) (end 145.05 86.71) (width 0.25) (layer F.Cu) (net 2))
 (segment (start 143.75 88.01) (end 145.05 88.01) (width 0.25) (layer F.Cu) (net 2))
 (segment (start 143.75 86.71) (end 143.75 88.01) (width 0.25) (layer F.Cu) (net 2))
 (segment (start 142.45 86.61) (end 143.65 86.61) (width 0.25) (layer F.Cu) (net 2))
 (segment (start 143.65 86.61) (end 143.75 86.71) (width 0.25) (layer F.Cu) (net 2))
 (segment (start 133.9 85.14) (end 135.75 85.14) (width 0.25) (layer B.Cu) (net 2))
 (segment (start 135.75 85.14) (end 136.6 85.99) (width 0.25) (layer B.Cu) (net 2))
 (segment (start 136.6 85.99) (end 136.6 86.14) (width 0.25) (layer B.Cu) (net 2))
 (segment (start 133.9 92.14) (end 133.9 85.14) (width 0.25) (layer B.Cu) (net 2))
 (segment (start 136.6 91.14) (end 136.6 91.29) (width 0.25) (layer B.Cu) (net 2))
 (segment (start 136.6 91.29) (end 135.75 92.14) (width 0.25) (layer B.Cu) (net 2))
 (segment (start 135.75 92.14) (end 134.925 92.14) (width 0.25) (layer B.Cu) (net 2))
 (segment (start 136.6 91.14) (end 136.6 89.94) (width 0.25) (layer F.Cu) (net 2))
 (segment (start 140.356109 86.295008) (end 138.965157 86.295008) (width 0.25) (layer F.Cu) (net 7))
 (segment (start 142.45 87.11) (end 141.171101 87.11) (width 0.25) (layer F.Cu) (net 7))
 (segment (start 138.395174 86.864991) (end 137.995175 87.26499) (width 0.25) (layer F.Cu) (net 7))
 (segment (start 141.171101 87.11) (end 140.356109 86.295008) (width 0.25) (layer F.Cu) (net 7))
 (segment (start 138.965157 86.295008) (end 138.395174 86.864991) (width 0.25) (layer F.Cu) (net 7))
 (segment (start 138.05 89.709998) (end 138.05 87.319815) (width 0.25) (layer B.Cu) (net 7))
 (segment (start 138.05 87.319815) (end 137.995175 87.26499) (width 0.25) (layer B.Cu) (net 7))
 (segment (start 136.6 88.64) (end 137.525 88.64) (width 0.25) (layer F.Cu) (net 7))
 (segment (start 137.525 88.64) (end 138.05 89.165) (width 0.25) (layer F.Cu) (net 7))
 (segment (start 138.05 89.165) (end 138.05 89.709998) (width 0.25) (layer F.Cu) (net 7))
 (via (at 138.05 89.709998) (size 0.8) (drill 0.4) (layers F.Cu B.Cu) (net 7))
 (segment (start 137.995175 87.365175) (end 137.995175 87.26499) (width 0.25) (layer B.Cu) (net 7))
 (segment (start 138.14 87.51) (end 137.995175 87.365175) (width 0.25) (layer B.Cu) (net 7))
 (via (at 137.995175 87.26499) (size 0.8) (drill 0.4) (layers F.Cu B.Cu) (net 7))
 (segment (start 142.43 87.09) (end 142.45 87.11) (width 0.25) (layer F.Cu) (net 7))
 (segment (start 139.471999 86.724999) (end 140.168001 86.724999) (width 0.25) (layer F.Cu) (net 6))
 (segment (start 141.053002 87.61) (end 141.775 87.61) (width 0.25) (layer F.Cu) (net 6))
 (segment (start 140.168001 86.724999) (end 141.053002 87.61) (width 0.25) (layer F.Cu) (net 6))
 (segment (start 138.606998 87.99) (end 139.054999 87.541999) (width 0.25) (layer F.Cu) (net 6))
 (segment (start 139.054999 87.141999) (end 139.471999 86.724999) (width 0.25) (layer F.Cu) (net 6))
 (segment (start 139.054999 87.541999) (end 139.054999 87.141999) (width 0.25) (layer F.Cu) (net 6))
 (segment (start 141.775 87.61) (end 142.45 87.61) (width 0.25) (layer F.Cu) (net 6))
 (segment (start 136.6 87.99) (end 138.606998 87.99) (width 0.25) (layer F.Cu) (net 6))
 (segment (start 148.79266 86.99) (end 148.392661 86.590001) (width 0.25) (layer B.Cu) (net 3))
 (segment (start 144.279664 86.590001) (end 142.750276 85.060613) (width 0.25) (layer B.Cu) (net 3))
 (segment (start 148.392661 86.590001) (end 144.279664 86.590001) (width 0.25) (layer B.Cu) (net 3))
 (segment (start 142.750276 85.060613) (end 142.350277 84.660614) (width 0.25) (layer B.Cu) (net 3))
 (segment (start 148.79266 86.17734) (end 148.79266 86.88) (width 0.25) (layer F.Cu) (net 3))
 (segment (start 148.79266 86.99) (end 148.79266 89.207658) (width 0.25) (layer F.Cu) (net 3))
 (segment (start 148.79266 86.88) (end 148.79266 86.99) (width 0.25) (layer F.Cu) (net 3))
 (via (at 148.79266 86.99) (size 0.8) (drill 0.4) (layers F.Cu B.Cu) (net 3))
 (segment (start 144.65 84.735) (end 144.287176 84.372176) (width 0.25) (layer F.Cu) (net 3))
 (via (at 142.350277 84.660614) (size 0.8) (drill 0.4) (layers F.Cu B.Cu) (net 3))
 (segment (start 144.287176 84.372176) (end 143.2044 84.372176) (width 0.25) (layer F.Cu) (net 3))
 (segment (start 144.65 85.41) (end 144.65 84.735) (width 0.25) (layer F.Cu) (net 3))
 (segment (start 143.2044 84.372176) (end 142.915962 84.660614) (width 0.25) (layer F.Cu) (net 3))
 (segment (start 142.915962 84.660614) (end 142.350277 84.660614) (width 0.25) (layer F.Cu) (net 3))
 (segment (start 148.79266 89.207658) (end 149.340003 89.755001) (width 0.25) (layer F.Cu) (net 3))
 (segment (start 152.200001 89.429999) (end 152.95 88.68) (width 0.25) (layer F.Cu) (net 3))
 (segment (start 149.340003 89.755001) (end 149.340003 89.760003) (width 0.25) (layer F.Cu) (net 3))
 (segment (start 149.340003 89.760003) (end 149.63 90.05) (width 0.25) (layer F.Cu) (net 3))
 (segment (start 149.63 90.05) (end 151.58 90.05) (width 0.25) (layer F.Cu) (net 3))
 (segment (start 151.58 90.05) (end 152.200001 89.429999) (width 0.25) (layer F.Cu) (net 3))
 (segment (start 150.1 84.87) (end 152.75 87.52) (width 0.25) (layer F.Cu) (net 3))
 (segment (start 152.75 87.52) (end 152.75 88.68) (width 0.25) (layer F.Cu) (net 3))
 (segment (start 150.1 84.87) (end 148.79266 86.17734) (width 0.25) (layer F.Cu) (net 3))
 (segment (start 145.998682 84.29651) (end 145.58849 84.29651) (width 0.25) (layer F.Cu) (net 4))
 (segment (start 145.15 84.735) (end 145.15 85.41) (width 0.25) (layer F.Cu) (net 4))
 (segment (start 147.56 84.87) (end 146.572172 84.87) (width 0.25) (layer F.Cu) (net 4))
 (segment (start 146.572172 84.87) (end 145.998682 84.29651) (width 0.25) (layer F.Cu) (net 4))
 (segment (start 145.58849 84.29651) (end 145.15 84.735) (width 0.25) (layer F.Cu) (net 4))
 (segment (start 151.05 88.68) (end 149.75141 88.68) (width 0.25) (layer F.Cu) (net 4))
 (segment (start 149.75141 88.68) (end 149.520866 88.910544) (width 0.25) (layer F.Cu) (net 4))
 (segment (start 149.519042 88.912368) (end 149.520866 88.910544) (width 0.25) (layer B.Cu) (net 4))
 (segment (start 149.502368 88.912368) (end 149.519042 88.912368) (width 0.25) (layer B.Cu) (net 4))
 (segment (start 149.52 88.67) (end 149.52 88.909678) (width 0.25) (layer B.Cu) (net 4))
 (segment (start 149.520866 88.344859) (end 149.520866 88.910544) (width 0.25) (layer B.Cu) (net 4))
 (segment (start 148.547828 84.87) (end 149.520866 85.843038) (width 0.25) (layer B.Cu) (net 4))
 (segment (start 149.519999 88.909677) (end 149.520866 88.910544) (width 0.25) (layer F.Cu) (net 4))
 (segment (start 147.56 84.87) (end 148.547828 84.87) (width 0.25) (layer B.Cu) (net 4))
 (via (at 149.520866 88.910544) (size 0.8) (drill 0.4) (layers F.Cu B.Cu) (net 4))
 (segment (start 149.52 88.909678) (end 149.520866 88.910544) (width 0.25) (layer B.Cu) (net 4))
 (segment (start 149.519999 88.670001) (end 149.519999 88.909677) (width 0.25) (layer F.Cu) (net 4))
 (segment (start 149.520866 85.843038) (end 149.520866 88.344859) (width 0.25) (layer B.Cu) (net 4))
 (segment (start 147.114694 90.365306) (end 147.54 89.94) (width 0.25) (layer F.Cu) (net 10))
 (segment (start 144.15 89.31) (end 144.15 89.970002) (width 0.25) (layer F.Cu) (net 10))
 (segment (start 144.545304 90.365306) (end 147.114694 90.365306) (width 0.25) (layer F.Cu) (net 10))
 (segment (start 144.15 89.970002) (end 144.545304 90.365306) (width 0.25) (layer F.Cu) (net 10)))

